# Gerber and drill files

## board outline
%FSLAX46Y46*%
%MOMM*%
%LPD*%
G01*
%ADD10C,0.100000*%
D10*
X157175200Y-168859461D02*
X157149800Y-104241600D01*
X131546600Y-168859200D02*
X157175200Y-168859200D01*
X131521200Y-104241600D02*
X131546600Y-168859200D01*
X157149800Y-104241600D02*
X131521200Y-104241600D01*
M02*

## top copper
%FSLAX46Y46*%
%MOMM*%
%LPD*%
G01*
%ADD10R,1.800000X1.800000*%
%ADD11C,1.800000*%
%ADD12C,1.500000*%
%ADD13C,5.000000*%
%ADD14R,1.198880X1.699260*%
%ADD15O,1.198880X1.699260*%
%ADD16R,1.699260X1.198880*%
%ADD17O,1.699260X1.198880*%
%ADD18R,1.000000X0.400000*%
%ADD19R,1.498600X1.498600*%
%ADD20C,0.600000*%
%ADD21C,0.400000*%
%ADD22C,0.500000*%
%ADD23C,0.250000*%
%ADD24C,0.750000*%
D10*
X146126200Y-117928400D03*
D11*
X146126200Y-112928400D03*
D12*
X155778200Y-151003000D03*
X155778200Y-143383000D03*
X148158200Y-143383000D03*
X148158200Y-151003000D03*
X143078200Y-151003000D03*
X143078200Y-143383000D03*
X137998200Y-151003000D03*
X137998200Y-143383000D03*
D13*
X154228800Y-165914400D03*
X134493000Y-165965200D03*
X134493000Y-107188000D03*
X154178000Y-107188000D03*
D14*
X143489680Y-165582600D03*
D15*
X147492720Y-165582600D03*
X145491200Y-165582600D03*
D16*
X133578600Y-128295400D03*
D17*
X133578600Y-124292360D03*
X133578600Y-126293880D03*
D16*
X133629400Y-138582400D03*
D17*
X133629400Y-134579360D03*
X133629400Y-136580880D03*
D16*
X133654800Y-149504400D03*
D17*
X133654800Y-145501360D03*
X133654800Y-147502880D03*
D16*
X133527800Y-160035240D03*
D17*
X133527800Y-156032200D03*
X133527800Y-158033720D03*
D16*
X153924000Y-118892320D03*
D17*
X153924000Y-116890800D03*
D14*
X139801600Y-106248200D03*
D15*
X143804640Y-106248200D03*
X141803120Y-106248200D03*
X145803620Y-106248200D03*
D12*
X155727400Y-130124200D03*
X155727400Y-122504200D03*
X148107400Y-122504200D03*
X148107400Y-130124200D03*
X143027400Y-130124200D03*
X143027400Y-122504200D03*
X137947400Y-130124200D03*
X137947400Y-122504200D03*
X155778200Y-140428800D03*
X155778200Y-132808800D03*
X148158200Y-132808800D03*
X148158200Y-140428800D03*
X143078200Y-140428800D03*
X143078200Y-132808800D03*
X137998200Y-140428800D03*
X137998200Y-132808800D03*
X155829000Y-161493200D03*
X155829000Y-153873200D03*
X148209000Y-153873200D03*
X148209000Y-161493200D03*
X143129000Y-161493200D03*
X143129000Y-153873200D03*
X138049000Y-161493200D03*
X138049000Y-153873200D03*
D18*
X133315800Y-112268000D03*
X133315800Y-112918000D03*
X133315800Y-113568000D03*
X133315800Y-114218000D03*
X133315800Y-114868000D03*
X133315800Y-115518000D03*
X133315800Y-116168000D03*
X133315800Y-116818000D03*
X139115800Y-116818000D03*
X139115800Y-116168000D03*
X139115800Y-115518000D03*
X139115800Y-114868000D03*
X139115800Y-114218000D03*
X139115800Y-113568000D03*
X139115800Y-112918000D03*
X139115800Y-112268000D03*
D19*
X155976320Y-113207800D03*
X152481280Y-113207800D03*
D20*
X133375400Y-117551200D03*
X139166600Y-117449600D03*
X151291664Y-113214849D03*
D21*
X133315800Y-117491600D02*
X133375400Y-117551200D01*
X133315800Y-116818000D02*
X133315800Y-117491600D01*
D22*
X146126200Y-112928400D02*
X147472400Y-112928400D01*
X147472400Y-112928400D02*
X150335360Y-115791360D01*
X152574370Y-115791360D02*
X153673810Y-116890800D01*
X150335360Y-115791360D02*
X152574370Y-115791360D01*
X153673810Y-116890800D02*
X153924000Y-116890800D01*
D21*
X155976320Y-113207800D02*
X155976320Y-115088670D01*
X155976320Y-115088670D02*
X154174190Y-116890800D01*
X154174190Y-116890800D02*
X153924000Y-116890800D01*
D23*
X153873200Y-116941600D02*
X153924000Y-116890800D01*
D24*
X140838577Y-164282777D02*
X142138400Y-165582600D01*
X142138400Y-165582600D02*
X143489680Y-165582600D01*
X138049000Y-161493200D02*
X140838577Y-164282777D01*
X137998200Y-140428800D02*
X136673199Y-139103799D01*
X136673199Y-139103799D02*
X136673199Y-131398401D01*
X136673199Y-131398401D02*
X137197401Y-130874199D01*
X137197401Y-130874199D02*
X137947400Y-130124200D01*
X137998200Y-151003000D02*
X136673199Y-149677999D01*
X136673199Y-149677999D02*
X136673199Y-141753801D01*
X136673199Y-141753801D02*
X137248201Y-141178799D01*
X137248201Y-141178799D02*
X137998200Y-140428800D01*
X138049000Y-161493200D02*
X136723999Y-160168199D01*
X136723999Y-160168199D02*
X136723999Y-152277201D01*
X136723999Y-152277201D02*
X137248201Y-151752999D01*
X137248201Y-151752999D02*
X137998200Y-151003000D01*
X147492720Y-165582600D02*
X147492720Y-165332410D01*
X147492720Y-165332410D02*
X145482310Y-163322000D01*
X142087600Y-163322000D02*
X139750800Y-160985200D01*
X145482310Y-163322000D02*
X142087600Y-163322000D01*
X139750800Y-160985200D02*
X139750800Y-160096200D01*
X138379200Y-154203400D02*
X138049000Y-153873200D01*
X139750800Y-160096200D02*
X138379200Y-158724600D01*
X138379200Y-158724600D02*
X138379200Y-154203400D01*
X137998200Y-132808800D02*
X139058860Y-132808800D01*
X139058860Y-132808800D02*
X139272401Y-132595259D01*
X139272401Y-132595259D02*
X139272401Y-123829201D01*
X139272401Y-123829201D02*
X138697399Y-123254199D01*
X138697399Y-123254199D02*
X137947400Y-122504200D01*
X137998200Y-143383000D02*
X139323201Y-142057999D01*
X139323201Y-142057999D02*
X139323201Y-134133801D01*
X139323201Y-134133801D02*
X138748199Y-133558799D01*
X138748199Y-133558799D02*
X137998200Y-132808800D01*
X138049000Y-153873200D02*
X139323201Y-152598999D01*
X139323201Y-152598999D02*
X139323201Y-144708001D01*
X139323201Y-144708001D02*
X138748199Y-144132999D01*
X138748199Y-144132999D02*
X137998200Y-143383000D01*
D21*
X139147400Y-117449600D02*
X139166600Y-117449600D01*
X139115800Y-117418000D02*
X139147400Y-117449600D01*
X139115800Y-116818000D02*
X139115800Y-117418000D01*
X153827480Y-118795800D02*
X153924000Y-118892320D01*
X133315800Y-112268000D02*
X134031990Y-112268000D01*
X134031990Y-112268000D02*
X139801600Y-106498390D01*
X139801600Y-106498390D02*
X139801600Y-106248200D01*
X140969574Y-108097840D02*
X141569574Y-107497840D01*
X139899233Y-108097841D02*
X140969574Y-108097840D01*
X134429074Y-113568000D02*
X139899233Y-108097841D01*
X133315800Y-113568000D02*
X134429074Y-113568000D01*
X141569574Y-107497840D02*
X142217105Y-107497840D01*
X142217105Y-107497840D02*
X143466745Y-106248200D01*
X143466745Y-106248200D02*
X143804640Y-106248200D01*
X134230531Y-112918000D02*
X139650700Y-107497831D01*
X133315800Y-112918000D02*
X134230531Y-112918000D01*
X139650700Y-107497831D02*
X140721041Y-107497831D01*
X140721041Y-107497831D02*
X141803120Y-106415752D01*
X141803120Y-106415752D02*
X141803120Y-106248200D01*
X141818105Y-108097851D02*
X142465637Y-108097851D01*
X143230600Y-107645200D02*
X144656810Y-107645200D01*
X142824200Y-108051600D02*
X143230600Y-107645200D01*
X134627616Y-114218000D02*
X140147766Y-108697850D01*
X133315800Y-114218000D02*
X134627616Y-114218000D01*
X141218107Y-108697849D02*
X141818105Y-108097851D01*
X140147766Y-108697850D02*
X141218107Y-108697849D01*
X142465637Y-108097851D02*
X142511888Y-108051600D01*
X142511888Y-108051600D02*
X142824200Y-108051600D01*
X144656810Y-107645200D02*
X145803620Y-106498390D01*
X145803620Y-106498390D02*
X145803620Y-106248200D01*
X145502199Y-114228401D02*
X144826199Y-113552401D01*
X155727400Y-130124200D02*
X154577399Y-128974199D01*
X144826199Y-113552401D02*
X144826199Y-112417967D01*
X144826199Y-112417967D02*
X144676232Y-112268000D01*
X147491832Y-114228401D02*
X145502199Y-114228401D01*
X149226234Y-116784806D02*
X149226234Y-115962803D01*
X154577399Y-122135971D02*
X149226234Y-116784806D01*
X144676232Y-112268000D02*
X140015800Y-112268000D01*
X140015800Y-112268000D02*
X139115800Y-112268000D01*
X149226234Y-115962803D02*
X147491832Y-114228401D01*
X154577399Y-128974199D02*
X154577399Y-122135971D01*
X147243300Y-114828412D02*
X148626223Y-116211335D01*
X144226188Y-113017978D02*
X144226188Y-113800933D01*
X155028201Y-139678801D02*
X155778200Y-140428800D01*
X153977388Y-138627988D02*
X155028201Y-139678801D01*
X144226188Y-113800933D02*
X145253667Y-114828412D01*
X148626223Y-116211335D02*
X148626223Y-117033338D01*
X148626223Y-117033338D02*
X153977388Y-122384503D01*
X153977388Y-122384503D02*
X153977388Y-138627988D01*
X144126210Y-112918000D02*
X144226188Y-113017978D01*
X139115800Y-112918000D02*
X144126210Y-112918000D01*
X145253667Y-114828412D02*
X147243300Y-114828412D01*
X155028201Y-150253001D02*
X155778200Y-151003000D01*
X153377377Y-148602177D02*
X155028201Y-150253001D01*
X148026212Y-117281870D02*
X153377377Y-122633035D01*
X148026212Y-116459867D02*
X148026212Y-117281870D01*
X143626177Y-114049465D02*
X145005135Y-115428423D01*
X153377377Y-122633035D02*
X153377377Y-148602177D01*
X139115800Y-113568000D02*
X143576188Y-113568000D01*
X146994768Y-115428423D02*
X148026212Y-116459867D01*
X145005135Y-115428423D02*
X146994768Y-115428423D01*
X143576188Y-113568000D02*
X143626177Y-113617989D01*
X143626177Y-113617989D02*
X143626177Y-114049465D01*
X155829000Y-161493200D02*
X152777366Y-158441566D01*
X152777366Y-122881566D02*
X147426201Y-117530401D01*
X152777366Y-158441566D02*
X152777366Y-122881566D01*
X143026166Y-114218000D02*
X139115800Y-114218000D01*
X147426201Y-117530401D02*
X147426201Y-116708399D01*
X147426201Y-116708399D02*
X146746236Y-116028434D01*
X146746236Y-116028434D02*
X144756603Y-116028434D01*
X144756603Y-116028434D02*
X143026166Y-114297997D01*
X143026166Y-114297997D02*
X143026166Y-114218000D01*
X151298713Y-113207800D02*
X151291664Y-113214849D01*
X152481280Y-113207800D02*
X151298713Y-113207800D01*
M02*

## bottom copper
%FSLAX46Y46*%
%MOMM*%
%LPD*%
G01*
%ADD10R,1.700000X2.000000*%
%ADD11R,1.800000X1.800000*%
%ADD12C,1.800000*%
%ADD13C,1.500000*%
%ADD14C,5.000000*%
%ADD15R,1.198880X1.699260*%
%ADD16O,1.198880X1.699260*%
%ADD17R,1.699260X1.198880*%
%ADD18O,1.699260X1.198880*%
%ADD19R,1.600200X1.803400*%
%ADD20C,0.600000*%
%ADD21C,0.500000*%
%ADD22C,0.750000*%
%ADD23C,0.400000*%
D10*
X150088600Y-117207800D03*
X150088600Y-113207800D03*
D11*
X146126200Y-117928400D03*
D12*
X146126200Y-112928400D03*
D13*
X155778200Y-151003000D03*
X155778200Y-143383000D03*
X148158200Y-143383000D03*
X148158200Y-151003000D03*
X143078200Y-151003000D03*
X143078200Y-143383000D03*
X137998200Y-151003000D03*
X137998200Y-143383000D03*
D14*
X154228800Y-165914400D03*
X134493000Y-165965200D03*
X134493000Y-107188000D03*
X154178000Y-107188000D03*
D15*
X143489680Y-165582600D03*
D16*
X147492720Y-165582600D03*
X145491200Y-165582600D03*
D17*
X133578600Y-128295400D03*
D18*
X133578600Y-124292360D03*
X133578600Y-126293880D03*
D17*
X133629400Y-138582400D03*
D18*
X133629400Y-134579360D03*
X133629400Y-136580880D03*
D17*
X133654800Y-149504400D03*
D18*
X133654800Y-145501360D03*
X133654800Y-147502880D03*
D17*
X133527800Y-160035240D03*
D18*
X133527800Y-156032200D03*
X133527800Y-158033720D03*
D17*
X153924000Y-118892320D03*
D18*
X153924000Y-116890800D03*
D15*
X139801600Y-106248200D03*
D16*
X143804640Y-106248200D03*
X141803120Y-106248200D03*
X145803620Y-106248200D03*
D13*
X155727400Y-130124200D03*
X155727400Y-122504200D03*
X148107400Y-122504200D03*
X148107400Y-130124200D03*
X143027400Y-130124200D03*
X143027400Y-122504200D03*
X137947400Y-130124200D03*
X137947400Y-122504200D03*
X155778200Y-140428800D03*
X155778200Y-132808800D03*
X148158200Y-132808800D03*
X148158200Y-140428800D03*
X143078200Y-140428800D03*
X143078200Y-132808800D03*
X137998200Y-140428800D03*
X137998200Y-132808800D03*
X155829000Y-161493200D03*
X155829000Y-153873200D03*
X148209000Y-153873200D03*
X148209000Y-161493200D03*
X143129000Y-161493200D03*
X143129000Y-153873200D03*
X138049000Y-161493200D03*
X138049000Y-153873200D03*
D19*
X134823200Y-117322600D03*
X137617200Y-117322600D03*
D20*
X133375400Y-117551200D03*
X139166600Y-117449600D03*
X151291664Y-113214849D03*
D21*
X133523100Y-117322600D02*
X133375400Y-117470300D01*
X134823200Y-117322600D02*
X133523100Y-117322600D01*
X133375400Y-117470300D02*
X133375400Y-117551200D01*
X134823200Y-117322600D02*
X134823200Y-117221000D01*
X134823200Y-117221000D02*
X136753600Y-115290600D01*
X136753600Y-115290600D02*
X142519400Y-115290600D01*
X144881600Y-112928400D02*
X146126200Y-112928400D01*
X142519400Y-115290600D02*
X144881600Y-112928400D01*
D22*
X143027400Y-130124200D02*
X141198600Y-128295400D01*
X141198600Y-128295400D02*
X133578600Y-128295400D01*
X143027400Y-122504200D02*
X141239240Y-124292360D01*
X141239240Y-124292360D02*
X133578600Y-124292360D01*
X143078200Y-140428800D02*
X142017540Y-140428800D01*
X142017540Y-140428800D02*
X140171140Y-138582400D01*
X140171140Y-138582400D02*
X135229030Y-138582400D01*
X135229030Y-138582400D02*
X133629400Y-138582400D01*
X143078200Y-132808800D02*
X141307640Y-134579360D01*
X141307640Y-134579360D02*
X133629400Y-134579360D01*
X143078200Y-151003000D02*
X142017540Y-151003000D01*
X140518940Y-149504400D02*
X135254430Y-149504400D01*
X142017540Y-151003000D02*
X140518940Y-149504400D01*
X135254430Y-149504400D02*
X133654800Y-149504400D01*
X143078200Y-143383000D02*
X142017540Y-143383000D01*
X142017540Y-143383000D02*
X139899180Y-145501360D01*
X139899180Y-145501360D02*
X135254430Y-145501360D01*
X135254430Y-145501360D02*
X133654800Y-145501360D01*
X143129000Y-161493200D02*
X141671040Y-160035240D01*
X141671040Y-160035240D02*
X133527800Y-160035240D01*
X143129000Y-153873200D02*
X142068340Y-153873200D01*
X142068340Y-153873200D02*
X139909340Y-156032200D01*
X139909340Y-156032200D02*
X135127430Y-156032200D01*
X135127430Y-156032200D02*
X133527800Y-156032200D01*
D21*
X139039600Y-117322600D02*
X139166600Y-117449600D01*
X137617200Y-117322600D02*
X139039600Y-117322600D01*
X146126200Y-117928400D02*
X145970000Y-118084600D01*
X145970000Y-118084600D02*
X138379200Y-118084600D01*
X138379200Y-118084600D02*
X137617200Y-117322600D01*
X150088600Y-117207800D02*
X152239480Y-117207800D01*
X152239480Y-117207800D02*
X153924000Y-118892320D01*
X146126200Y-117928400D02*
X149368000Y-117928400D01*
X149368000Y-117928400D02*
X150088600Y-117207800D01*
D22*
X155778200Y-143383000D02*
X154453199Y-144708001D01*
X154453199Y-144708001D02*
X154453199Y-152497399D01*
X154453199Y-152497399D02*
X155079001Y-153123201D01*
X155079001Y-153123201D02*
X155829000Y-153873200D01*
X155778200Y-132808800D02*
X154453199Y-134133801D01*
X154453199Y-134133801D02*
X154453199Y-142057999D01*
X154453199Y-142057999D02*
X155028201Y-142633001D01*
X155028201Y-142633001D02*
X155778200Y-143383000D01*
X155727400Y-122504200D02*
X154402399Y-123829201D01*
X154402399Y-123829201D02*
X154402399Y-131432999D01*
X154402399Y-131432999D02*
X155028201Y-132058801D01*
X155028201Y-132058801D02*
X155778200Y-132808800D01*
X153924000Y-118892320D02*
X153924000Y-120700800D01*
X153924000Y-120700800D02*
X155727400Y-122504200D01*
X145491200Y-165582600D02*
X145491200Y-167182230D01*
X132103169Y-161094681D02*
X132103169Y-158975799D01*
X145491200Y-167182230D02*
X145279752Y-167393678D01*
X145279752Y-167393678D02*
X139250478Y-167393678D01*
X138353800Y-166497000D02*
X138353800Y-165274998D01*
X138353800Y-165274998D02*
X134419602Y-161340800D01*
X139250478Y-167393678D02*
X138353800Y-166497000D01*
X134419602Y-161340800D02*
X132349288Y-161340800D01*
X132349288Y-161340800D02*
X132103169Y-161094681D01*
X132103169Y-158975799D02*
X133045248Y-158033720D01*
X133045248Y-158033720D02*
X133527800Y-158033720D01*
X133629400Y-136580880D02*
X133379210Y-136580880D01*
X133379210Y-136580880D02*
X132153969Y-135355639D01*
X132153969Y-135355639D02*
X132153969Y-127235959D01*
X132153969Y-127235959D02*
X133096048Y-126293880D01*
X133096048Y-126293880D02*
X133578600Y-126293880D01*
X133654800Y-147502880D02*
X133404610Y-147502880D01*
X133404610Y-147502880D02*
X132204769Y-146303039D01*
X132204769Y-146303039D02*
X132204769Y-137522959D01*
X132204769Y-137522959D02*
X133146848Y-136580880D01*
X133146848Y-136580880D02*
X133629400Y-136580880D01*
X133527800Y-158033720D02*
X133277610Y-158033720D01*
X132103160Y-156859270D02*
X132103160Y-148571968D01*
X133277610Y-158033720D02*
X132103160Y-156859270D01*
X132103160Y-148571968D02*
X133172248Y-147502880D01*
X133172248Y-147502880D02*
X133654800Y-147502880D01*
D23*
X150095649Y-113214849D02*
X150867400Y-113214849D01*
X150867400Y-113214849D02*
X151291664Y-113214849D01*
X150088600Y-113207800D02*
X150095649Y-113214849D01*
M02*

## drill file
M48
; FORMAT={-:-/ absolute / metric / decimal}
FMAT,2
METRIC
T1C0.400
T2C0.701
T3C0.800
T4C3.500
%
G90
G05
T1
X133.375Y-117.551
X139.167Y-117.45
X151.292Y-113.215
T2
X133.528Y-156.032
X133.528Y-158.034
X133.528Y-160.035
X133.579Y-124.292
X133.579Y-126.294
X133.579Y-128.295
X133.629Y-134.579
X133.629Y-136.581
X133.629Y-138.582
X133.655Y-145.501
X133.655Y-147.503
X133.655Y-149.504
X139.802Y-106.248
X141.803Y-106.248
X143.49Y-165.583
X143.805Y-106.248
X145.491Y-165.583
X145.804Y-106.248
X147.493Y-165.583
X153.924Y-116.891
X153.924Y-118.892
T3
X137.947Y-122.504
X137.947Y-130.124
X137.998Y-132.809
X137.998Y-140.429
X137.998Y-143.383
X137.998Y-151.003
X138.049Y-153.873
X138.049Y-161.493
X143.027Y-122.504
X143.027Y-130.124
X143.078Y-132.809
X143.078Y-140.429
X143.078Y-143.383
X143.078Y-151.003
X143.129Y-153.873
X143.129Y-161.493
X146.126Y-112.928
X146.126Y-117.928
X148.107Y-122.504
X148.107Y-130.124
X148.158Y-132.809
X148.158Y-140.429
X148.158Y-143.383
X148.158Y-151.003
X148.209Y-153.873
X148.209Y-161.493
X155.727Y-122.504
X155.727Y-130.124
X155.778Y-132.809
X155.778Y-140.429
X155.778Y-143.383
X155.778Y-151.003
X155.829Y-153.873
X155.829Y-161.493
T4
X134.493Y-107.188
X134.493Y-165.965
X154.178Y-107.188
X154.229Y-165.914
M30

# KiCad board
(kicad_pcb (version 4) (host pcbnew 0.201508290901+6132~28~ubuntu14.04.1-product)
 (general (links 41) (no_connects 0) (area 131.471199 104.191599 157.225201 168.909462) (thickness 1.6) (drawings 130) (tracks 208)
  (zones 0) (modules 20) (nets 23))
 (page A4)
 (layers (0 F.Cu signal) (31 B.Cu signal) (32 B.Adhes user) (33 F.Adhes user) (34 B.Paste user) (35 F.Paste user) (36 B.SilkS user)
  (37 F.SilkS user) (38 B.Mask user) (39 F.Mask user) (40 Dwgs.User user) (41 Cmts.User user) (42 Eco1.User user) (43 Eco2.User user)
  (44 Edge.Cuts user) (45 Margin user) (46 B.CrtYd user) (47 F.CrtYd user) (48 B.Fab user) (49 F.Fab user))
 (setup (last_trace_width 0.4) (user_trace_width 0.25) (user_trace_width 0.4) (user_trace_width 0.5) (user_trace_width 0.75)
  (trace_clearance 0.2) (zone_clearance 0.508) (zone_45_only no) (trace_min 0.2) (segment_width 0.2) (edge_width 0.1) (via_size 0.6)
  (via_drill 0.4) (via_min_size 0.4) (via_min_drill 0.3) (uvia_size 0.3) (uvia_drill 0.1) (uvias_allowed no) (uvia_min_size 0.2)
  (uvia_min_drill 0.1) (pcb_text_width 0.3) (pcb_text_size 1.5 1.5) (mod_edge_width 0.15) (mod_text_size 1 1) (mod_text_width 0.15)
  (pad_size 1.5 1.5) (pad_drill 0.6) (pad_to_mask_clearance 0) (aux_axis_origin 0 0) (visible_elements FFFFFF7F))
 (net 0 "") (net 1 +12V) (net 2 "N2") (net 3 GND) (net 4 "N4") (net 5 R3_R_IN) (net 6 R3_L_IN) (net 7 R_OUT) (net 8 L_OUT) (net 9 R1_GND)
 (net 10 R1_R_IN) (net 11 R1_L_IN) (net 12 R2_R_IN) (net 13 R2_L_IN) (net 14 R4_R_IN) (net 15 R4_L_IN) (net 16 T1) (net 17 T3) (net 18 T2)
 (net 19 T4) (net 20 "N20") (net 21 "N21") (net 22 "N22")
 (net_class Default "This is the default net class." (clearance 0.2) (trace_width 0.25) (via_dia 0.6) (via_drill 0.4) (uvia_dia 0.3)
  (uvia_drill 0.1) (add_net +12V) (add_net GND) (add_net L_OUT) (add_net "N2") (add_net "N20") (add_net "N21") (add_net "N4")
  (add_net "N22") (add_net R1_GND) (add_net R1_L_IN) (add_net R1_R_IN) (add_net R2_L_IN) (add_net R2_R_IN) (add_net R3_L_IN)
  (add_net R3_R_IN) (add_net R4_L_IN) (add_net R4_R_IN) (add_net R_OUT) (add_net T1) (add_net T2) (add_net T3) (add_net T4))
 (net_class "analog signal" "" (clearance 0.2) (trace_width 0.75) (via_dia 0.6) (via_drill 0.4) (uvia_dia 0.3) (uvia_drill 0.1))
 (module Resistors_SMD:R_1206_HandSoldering (layer B.Cu) (at 150.0886 115.2078 90)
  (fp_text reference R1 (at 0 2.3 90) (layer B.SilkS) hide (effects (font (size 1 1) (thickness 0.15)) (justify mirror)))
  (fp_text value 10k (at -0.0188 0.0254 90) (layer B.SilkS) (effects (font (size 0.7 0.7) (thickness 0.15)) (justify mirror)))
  (pad 1 smd rect (at -2 0 90) (size 2 1.7) (layers B.Cu B.Paste B.Mask) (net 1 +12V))
  (pad 2 smd rect (at 2 0 90) (size 2 1.7) (layers B.Cu B.Paste B.Mask) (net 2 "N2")))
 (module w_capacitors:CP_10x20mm (layer F.Cu) (at 146.1262 115.4284)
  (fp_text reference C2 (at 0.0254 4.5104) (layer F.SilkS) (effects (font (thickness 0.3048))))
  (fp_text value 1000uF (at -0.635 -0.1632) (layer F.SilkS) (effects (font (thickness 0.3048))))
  (pad 1 thru_hole rect (at 0 2.5) (size 1.8 1.8) (drill 0.8) (layers *.Cu *.Mask F.SilkS) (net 1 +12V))
  (pad 2 thru_hole circle (at 0 -2.5) (size 1.8 1.8) (drill 0.8) (layers *.Cu *.Mask F.SilkS) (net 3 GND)))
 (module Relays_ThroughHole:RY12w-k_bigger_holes (layer F.Cu) (at 156.9782 152.103 180)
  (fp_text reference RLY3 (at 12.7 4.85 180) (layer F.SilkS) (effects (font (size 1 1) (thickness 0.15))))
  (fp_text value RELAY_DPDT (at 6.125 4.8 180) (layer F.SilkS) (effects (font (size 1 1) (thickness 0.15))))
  (pad 1 thru_hole circle (at 1.2 1.1 180) (size 1.5 1.5) (drill 0.8) (layers *.Cu *.Mask F.SilkS) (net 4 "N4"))
  (pad 8 thru_hole circle (at 1.2 8.72 180) (size 1.5 1.5) (drill 0.8) (layers *.Cu *.Mask F.SilkS) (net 1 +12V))
  (pad 7 thru_hole circle (at 8.82 8.72 180) (size 1.5 1.5) (drill 0.8) (layers *.Cu *.Mask F.SilkS))
  (pad 2 thru_hole circle (at 8.82 1.1 180) (size 1.5 1.5) (drill 0.8) (layers *.Cu *.Mask F.SilkS))
  (pad 3 thru_hole circle (at 13.9 1.1 180) (size 1.5 1.5) (drill 0.8) (layers *.Cu *.Mask F.SilkS) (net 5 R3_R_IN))
  (pad 6 thru_hole circle (at 13.9 8.72 180) (size 1.5 1.5) (drill 0.8) (layers *.Cu *.Mask F.SilkS) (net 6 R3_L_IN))
  (pad 4 thru_hole circle (at 18.98 1.1 180) (size 1.5 1.5) (drill 0.8) (layers *.Cu *.Mask F.SilkS) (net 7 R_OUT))
  (pad 5 thru_hole circle (at 18.98 8.72 180) (size 1.5 1.5) (drill 0.8) (layers *.Cu *.Mask F.SilkS) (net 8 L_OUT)))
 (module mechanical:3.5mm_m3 (layer F.Cu) (at 154.2288 166.0144)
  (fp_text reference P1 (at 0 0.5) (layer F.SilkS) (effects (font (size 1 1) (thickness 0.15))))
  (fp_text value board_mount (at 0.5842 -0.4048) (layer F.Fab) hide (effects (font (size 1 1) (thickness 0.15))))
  (pad 1 thru_hole circle (at 0 -0.1) (size 5 5) (drill 3.5) (layers *.Cu *.Mask F.SilkS)))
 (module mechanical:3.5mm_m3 (layer F.Cu) (at 134.493 166.0652)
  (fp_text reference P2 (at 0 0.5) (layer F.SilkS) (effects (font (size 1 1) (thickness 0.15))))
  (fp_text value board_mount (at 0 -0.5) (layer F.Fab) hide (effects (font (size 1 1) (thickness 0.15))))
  (pad 1 thru_hole circle (at 0 -0.1) (size 5 5) (drill 3.5) (layers *.Cu *.Mask F.SilkS)))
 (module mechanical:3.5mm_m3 (layer F.Cu) (at 134.493 107.288)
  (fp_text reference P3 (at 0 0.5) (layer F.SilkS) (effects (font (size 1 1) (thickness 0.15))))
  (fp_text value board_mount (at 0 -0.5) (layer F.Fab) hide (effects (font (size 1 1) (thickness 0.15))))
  (pad 1 thru_hole circle (at 0 -0.1) (size 5 5) (drill 3.5) (layers *.Cu *.Mask F.SilkS)))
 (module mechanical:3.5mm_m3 (layer F.Cu) (at 154.178 107.288)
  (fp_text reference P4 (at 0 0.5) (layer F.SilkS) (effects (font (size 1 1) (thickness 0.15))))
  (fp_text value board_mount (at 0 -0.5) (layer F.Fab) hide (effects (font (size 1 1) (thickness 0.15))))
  (pad 1 thru_hole circle (at 0 -0.1) (size 5 5) (drill 3.5) (layers *.Cu *.Mask F.SilkS)))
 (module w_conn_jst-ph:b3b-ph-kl (layer F.Cu) (at 145.4912 165.5826)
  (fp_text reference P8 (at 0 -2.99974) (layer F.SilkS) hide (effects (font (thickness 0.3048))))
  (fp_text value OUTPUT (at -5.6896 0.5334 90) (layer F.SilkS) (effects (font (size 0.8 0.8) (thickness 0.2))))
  (pad 1 thru_hole rect (at -2.00152 0) (size 1.19888 1.69926) (drill 0.70104) (layers *.Cu *.Mask F.SilkS) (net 7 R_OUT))
  (pad 3 thru_hole oval (at 2.00152 0) (size 1.19888 1.69926) (drill 0.70104) (layers *.Cu *.Mask F.SilkS) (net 8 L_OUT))
  (pad 2 thru_hole oval (at 0 0) (size 1.19888 1.69926) (drill 0.70104) (layers *.Cu *.Mask F.SilkS) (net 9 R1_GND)))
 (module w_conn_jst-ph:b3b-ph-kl (layer F.Cu) (at 133.5786 126.29388 90)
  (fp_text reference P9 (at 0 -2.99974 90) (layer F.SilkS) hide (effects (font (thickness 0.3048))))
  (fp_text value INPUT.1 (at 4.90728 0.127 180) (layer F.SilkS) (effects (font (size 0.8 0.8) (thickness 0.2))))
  (pad 1 thru_hole rect (at -2.00152 0 90) (size 1.19888 1.69926) (drill 0.70104) (layers *.Cu *.Mask F.SilkS) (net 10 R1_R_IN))
  (pad 3 thru_hole oval (at 2.00152 0 90) (size 1.19888 1.69926) (drill 0.70104) (layers *.Cu *.Mask F.SilkS) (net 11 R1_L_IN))
  (pad 2 thru_hole oval (at 0 0 90) (size 1.19888 1.69926) (drill 0.70104) (layers *.Cu *.Mask F.SilkS) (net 9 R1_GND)))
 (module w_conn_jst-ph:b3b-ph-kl (layer F.Cu) (at 133.6294 136.58088 90)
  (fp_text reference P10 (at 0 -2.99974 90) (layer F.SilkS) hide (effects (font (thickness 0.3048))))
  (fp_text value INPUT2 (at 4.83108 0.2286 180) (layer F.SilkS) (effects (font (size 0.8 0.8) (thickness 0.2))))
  (pad 1 thru_hole rect (at -2.00152 0 90) (size 1.19888 1.69926) (drill 0.70104) (layers *.Cu *.Mask F.SilkS) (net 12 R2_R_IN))
  (pad 3 thru_hole oval (at 2.00152 0 90) (size 1.19888 1.69926) (drill 0.70104) (layers *.Cu *.Mask F.SilkS) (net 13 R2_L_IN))
  (pad 2 thru_hole oval (at 0 0 90) (size 1.19888 1.69926) (drill 0.70104) (layers *.Cu *.Mask F.SilkS) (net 9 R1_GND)))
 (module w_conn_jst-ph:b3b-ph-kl (layer F.Cu) (at 133.6548 147.50288 90)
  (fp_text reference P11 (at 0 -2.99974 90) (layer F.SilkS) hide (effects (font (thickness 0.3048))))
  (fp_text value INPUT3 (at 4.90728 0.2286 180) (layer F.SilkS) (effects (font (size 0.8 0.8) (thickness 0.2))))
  (pad 1 thru_hole rect (at -2.00152 0 90) (size 1.19888 1.69926) (drill 0.70104) (layers *.Cu *.Mask F.SilkS) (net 5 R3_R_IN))
  (pad 3 thru_hole oval (at 2.00152 0 90) (size 1.19888 1.69926) (drill 0.70104) (layers *.Cu *.Mask F.SilkS) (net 6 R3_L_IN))
  (pad 2 thru_hole oval (at 0 0 90) (size 1.19888 1.69926) (drill 0.70104) (layers *.Cu *.Mask F.SilkS) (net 9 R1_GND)))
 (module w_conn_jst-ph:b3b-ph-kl (layer F.Cu) (at 133.5278 158.03372 90)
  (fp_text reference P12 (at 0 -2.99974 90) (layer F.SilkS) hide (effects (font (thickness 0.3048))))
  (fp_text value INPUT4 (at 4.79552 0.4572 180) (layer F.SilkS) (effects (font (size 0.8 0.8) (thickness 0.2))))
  (pad 1 thru_hole rect (at -2.00152 0 90) (size 1.19888 1.69926) (drill 0.70104) (layers *.Cu *.Mask F.SilkS) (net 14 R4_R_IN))
  (pad 3 thru_hole oval (at 2.00152 0 90) (size 1.19888 1.69926) (drill 0.70104) (layers *.Cu *.Mask F.SilkS) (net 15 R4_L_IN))
  (pad 2 thru_hole oval (at 0 0 90) (size 1.19888 1.69926) (drill 0.70104) (layers *.Cu *.Mask F.SilkS) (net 9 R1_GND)))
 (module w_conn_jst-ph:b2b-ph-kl (layer F.Cu) (at 153.924 117.89156 90)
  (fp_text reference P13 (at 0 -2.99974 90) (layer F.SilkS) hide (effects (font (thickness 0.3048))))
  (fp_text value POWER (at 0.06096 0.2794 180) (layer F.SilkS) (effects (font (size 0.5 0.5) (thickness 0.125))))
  (pad 1 thru_hole rect (at -1.00076 0 90) (size 1.19888 1.69926) (drill 0.70104) (layers *.Cu *.Mask F.SilkS) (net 1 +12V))
  (pad 2 thru_hole oval (at 1.00076 0 90) (size 1.19888 1.69926) (drill 0.70104) (layers *.Cu *.Mask F.SilkS) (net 3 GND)))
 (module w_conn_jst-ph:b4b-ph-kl (layer F.Cu) (at 142.80388 106.2482)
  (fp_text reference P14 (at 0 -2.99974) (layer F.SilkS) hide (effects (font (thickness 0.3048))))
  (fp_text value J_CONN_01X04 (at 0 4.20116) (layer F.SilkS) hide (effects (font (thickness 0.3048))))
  (pad 1 thru_hole rect (at -3.00228 0) (size 1.19888 1.69926) (drill 0.70104) (layers *.Cu *.Mask F.SilkS) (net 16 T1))
  (pad 3 thru_hole oval (at 1.00076 0) (size 1.19888 1.69926) (drill 0.70104) (layers *.Cu *.Mask F.SilkS) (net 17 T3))
  (pad 2 thru_hole oval (at -1.00076 0) (size 1.19888 1.69926) (drill 0.70104) (layers *.Cu *.Mask F.SilkS) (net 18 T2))
  (pad 4 thru_hole oval (at 2.99974 0) (size 1.19888 1.69926) (drill 0.70104) (layers *.Cu *.Mask F.SilkS) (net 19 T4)))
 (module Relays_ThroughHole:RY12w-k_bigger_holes (layer F.Cu) (at 156.9274 131.2242 180)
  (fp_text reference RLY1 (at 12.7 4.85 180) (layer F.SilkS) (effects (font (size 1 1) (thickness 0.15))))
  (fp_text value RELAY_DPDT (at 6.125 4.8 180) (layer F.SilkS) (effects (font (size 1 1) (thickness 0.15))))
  (pad 1 thru_hole circle (at 1.2 1.1 180) (size 1.5 1.5) (drill 0.8) (layers *.Cu *.Mask F.SilkS) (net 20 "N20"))
  (pad 8 thru_hole circle (at 1.2 8.72 180) (size 1.5 1.5) (drill 0.8) (layers *.Cu *.Mask F.SilkS) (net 1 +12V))
  (pad 7 thru_hole circle (at 8.82 8.72 180) (size 1.5 1.5) (drill 0.8) (layers *.Cu *.Mask F.SilkS))
  (pad 2 thru_hole circle (at 8.82 1.1 180) (size 1.5 1.5) (drill 0.8) (layers *.Cu *.Mask F.SilkS))
  (pad 3 thru_hole circle (at 13.9 1.1 180) (size 1.5 1.5) (drill 0.8) (layers *.Cu *.Mask F.SilkS) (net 10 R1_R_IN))
  (pad 6 thru_hole circle (at 13.9 8.72 180) (size 1.5 1.5) (drill 0.8) (layers *.Cu *.Mask F.SilkS) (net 11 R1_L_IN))
  (pad 4 thru_hole circle (at 18.98 1.1 180) (size 1.5 1.5) (drill 0.8) (layers *.Cu *.Mask F.SilkS) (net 7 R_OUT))
  (pad 5 thru_hole circle (at 18.98 8.72 180) (size 1.5 1.5) (drill 0.8) (layers *.Cu *.Mask F.SilkS) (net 8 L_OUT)))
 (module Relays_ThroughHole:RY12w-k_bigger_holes (layer F.Cu) (at 156.9782 141.5288 180)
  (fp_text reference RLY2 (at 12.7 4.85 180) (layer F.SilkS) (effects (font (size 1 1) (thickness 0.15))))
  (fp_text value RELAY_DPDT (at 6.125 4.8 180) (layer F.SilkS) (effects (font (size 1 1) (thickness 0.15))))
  (pad 1 thru_hole circle (at 1.2 1.1 180) (size 1.5 1.5) (drill 0.8) (layers *.Cu *.Mask F.SilkS) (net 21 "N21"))
  (pad 8 thru_hole circle (at 1.2 8.72 180) (size 1.5 1.5) (drill 0.8) (layers *.Cu *.Mask F.SilkS) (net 1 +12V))
  (pad 7 thru_hole circle (at 8.82 8.72 180) (size 1.5 1.5) (drill 0.8) (layers *.Cu *.Mask F.SilkS))
  (pad 2 thru_hole circle (at 8.82 1.1 180) (size 1.5 1.5) (drill 0.8) (layers *.Cu *.Mask F.SilkS))
  (pad 3 thru_hole circle (at 13.9 1.1 180) (size 1.5 1.5) (drill 0.8) (layers *.Cu *.Mask F.SilkS) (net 12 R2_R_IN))
  (pad 6 thru_hole circle (at 13.9 8.72 180) (size 1.5 1.5) (drill 0.8) (layers *.Cu *.Mask F.SilkS) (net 13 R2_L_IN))
  (pad 4 thru_hole circle (at 18.98 1.1 180) (size 1.5 1.5) (drill 0.8) (layers *.Cu *.Mask F.SilkS) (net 7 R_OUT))
  (pad 5 thru_hole circle (at 18.98 8.72 180) (size 1.5 1.5) (drill 0.8) (layers *.Cu *.Mask F.SilkS) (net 8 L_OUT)))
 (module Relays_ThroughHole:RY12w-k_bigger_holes (layer F.Cu) (at 157.029 162.5932 180)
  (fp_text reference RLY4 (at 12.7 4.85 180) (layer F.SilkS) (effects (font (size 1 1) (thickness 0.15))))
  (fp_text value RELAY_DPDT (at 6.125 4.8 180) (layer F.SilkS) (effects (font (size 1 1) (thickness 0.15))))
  (pad 1 thru_hole circle (at 1.2 1.1 180) (size 1.5 1.5) (drill 0.8) (layers *.Cu *.Mask F.SilkS) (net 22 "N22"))
  (pad 8 thru_hole circle (at 1.2 8.72 180) (size 1.5 1.5) (drill 0.8) (layers *.Cu *.Mask F.SilkS) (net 1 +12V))
  (pad 7 thru_hole circle (at 8.82 8.72 180) (size 1.5 1.5) (drill 0.8) (layers *.Cu *.Mask F.SilkS))
  (pad 2 thru_hole circle (at 8.82 1.1 180) (size 1.5 1.5) (drill 0.8) (layers *.Cu *.Mask F.SilkS))
  (pad 3 thru_hole circle (at 13.9 1.1 180) (size 1.5 1.5) (drill 0.8) (layers *.Cu *.Mask F.SilkS) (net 14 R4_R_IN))
  (pad 6 thru_hole circle (at 13.9 8.72 180) (size 1.5 1.5) (drill 0.8) (layers *.Cu *.Mask F.SilkS) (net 15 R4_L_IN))
  (pad 4 thru_hole circle (at 18.98 1.1 180) (size 1.5 1.5) (drill 0.8) (layers *.Cu *.Mask F.SilkS) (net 7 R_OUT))
  (pad 5 thru_hole circle (at 18.98 8.72 180) (size 1.5 1.5) (drill 0.8) (layers *.Cu *.Mask F.SilkS) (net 8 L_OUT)))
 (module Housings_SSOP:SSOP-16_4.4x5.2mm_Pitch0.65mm (layer F.Cu) (at 136.2158 114.543)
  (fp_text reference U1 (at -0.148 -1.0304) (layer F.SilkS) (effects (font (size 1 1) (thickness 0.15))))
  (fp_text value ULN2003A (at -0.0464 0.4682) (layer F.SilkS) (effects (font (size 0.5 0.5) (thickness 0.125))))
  (pad 1 smd rect (at -2.9 -2.275) (size 1 0.4) (layers F.Cu F.Paste F.Mask) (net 16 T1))
  (pad 2 smd rect (at -2.9 -1.625) (size 1 0.4) (layers F.Cu F.Paste F.Mask) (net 18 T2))
  (pad 3 smd rect (at -2.9 -0.975) (size 1 0.4) (layers F.Cu F.Paste F.Mask) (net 17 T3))
  (pad 4 smd rect (at -2.9 -0.325) (size 1 0.4) (layers F.Cu F.Paste F.Mask) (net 19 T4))
  (pad 5 smd rect (at -2.9 0.325) (size 1 0.4) (layers F.Cu F.Paste F.Mask))
  (pad 6 smd rect (at -2.9 0.975) (size 1 0.4) (layers F.Cu F.Paste F.Mask))
  (pad 7 smd rect (at -2.9 1.625) (size 1 0.4) (layers F.Cu F.Paste F.Mask))
  (pad 8 smd rect (at -2.9 2.275) (size 1 0.4) (layers F.Cu F.Paste F.Mask) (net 3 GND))
  (pad 9 smd rect (at 2.9 2.275) (size 1 0.4) (layers F.Cu F.Paste F.Mask) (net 1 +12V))
  (pad 10 smd rect (at 2.9 1.625) (size 1 0.4) (layers F.Cu F.Paste F.Mask))
  (pad 11 smd rect (at 2.9 0.975) (size 1 0.4) (layers F.Cu F.Paste F.Mask))
  (pad 12 smd rect (at 2.9 0.325) (size 1 0.4) (layers F.Cu F.Paste F.Mask))
  (pad 13 smd rect (at 2.9 -0.325) (size 1 0.4) (layers F.Cu F.Paste F.Mask) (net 22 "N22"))
  (pad 14 smd rect (at 2.9 -0.975) (size 1 0.4) (layers F.Cu F.Paste F.Mask) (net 4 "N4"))
  (pad 15 smd rect (at 2.9 -1.625) (size 1 0.4) (layers F.Cu F.Paste F.Mask) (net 21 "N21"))
  (pad 16 smd rect (at 2.9 -2.275) (size 1 0.4) (layers F.Cu F.Paste F.Mask) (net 20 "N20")))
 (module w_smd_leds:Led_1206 (layer F.Cu) (at 154.2288 113.2078 180)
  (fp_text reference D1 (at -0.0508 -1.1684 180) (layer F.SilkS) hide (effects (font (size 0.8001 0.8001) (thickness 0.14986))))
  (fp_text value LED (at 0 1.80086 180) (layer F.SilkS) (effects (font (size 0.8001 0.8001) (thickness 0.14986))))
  (pad 1 smd rect (at -1.74752 0 180) (size 1.4986 1.4986) (layers F.Cu F.Paste F.Mask) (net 3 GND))
  (pad 2 smd rect (at 1.74752 0 180) (size 1.4986 1.4986) (layers F.Cu F.Paste F.Mask) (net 2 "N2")))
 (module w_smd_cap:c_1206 (layer B.Cu) (at 136.2202 117.3226 180)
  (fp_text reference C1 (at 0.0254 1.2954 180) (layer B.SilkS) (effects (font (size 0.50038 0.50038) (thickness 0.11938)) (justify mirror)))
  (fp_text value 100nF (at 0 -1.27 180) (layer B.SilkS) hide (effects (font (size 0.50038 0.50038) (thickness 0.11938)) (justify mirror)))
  (pad 1 smd rect (at 1.397 0 180) (size 1.6002 1.8034) (layers B.Cu B.Paste B.Mask) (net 3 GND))
  (pad 2 smd rect (at -1.397 0 180) (size 1.6002 1.8034) (layers B.Cu B.Paste B.Mask) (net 1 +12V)))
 (gr_line (start 157.1752 168.859461) (end 157.1498 104.2416) (layer Edge.Cuts) (width 0.1))
 (gr_line (start 131.5466 168.8592) (end 157.1752 168.8592) (layer Edge.Cuts) (width 0.1))
 (gr_line (start 131.5212 104.2416) (end 131.5466 168.8592) (layer Edge.Cuts) (width 0.1))
 (gr_line (start 157.1498 104.2416) (end 131.5212 104.2416) (layer Edge.Cuts) (width 0.1))
 (segment (start 133.3158 117.4916) (end 133.3754 117.5512) (width 0.4) (layer F.Cu) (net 3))
 (segment (start 133.3158 116.818) (end 133.3158 117.4916) (width 0.4) (layer F.Cu) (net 3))
 (segment (start 133.5231 117.3226) (end 133.3754 117.4703) (width 0.5) (layer B.Cu) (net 3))
 (segment (start 134.8232 117.3226) (end 133.5231 117.3226) (width 0.5) (layer B.Cu) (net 3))
 (segment (start 133.3754 117.4703) (end 133.3754 117.5512) (width 0.5) (layer B.Cu) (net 3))
 (segment (start 134.8232 117.3226) (end 134.8232 117.221) (width 0.5) (layer B.Cu) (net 3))
 (segment (start 134.8232 117.221) (end 136.7536 115.2906) (width 0.5) (layer B.Cu) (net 3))
 (segment (start 136.7536 115.2906) (end 142.5194 115.2906) (width 0.5) (layer B.Cu) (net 3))
 (segment (start 144.8816 112.9284) (end 146.1262 112.9284) (width 0.5) (layer B.Cu) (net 3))
 (segment (start 142.5194 115.2906) (end 144.8816 112.9284) (width 0.5) (layer B.Cu) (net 3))
 (segment (start 146.1262 112.9284) (end 147.4724 112.9284) (width 0.5) (layer F.Cu) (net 3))
 (segment (start 147.4724 112.9284) (end 150.33536 115.79136) (width 0.5) (layer F.Cu) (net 3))
 (segment (start 152.57437 115.79136) (end 153.67381 116.8908) (width 0.5) (layer F.Cu) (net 3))
 (segment (start 150.33536 115.79136) (end 152.57437 115.79136) (width 0.5) (layer F.Cu) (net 3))
 (segment (start 153.67381 116.8908) (end 153.924 116.8908) (width 0.5) (layer F.Cu) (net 3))
 (segment (start 155.97632 113.2078) (end 155.97632 115.08867) (width 0.4) (layer F.Cu) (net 3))
 (segment (start 155.97632 115.08867) (end 154.17419 116.8908) (width 0.4) (layer F.Cu) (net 3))
 (segment (start 154.17419 116.8908) (end 153.924 116.8908) (width 0.4) (layer F.Cu) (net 3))
 (segment (start 153.8732 116.9416) (end 153.924 116.8908) (width 0.25) (layer F.Cu) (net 3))
 (segment (start 140.838577 164.282777) (end 142.1384 165.5826) (width 0.75) (layer F.Cu) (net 7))
 (segment (start 142.1384 165.5826) (end 143.48968 165.5826) (width 0.75) (layer F.Cu) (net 7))
 (segment (start 138.049 161.4932) (end 140.838577 164.282777) (width 0.75) (layer F.Cu) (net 7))
 (segment (start 137.9982 140.4288) (end 136.673199 139.103799) (width 0.75) (layer F.Cu) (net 7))
 (segment (start 136.673199 139.103799) (end 136.673199 131.398401) (width 0.75) (layer F.Cu) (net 7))
 (segment (start 136.673199 131.398401) (end 137.197401 130.874199) (width 0.75) (layer F.Cu) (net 7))
 (segment (start 137.197401 130.874199) (end 137.9474 130.1242) (width 0.75) (layer F.Cu) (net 7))
 (segment (start 137.9982 151.003) (end 136.673199 149.677999) (width 0.75) (layer F.Cu) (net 7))
 (segment (start 136.673199 149.677999) (end 136.673199 141.753801) (width 0.75) (layer F.Cu) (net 7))
 (segment (start 136.673199 141.753801) (end 137.248201 141.178799) (width 0.75) (layer F.Cu) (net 7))
 (segment (start 137.248201 141.178799) (end 137.9982 140.4288) (width 0.75) (layer F.Cu) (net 7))
 (segment (start 138.049 161.4932) (end 136.723999 160.168199) (width 0.75) (layer F.Cu) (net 7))
 (segment (start 136.723999 160.168199) (end 136.723999 152.277201) (width 0.75) (layer F.Cu) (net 7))
 (segment (start 136.723999 152.277201) (end 137.248201 151.752999) (width 0.75) (layer F.Cu) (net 7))
 (segment (start 137.248201 151.752999) (end 137.9982 151.003) (width 0.75) (layer F.Cu) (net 7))
 (segment (start 147.49272 165.5826) (end 147.49272 165.33241) (width 0.75) (layer F.Cu) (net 8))
 (segment (start 147.49272 165.33241) (end 145.48231 163.322) (width 0.75) (layer F.Cu) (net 8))
 (segment (start 142.0876 163.322) (end 139.7508 160.9852) (width 0.75) (layer F.Cu) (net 8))
 (segment (start 145.48231 163.322) (end 142.0876 163.322) (width 0.75) (layer F.Cu) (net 8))
 (segment (start 139.7508 160.9852) (end 139.7508 160.0962) (width 0.75) (layer F.Cu) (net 8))
 (segment (start 138.3792 154.2034) (end 138.049 153.8732) (width 0.75) (layer F.Cu) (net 8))
 (segment (start 139.7508 160.0962) (end 138.3792 158.7246) (width 0.75) (layer F.Cu) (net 8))
 (segment (start 138.3792 158.7246) (end 138.3792 154.2034) (width 0.75) (layer F.Cu) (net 8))
 (segment (start 137.9982 132.8088) (end 139.05886 132.8088) (width 0.75) (layer F.Cu) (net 8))
 (segment (start 139.05886 132.8088) (end 139.272401 132.595259) (width 0.75) (layer F.Cu) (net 8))
 (segment (start 139.272401 132.595259) (end 139.272401 123.829201) (width 0.75) (layer F.Cu) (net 8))
 (segment (start 139.272401 123.829201) (end 138.697399 123.254199) (width 0.75) (layer F.Cu) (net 8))
 (segment (start 138.697399 123.254199) (end 137.9474 122.5042) (width 0.75) (layer F.Cu) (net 8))
 (segment (start 137.9982 143.383) (end 139.323201 142.057999) (width 0.75) (layer F.Cu) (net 8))
 (segment (start 139.323201 142.057999) (end 139.323201 134.133801) (width 0.75) (layer F.Cu) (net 8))
 (segment (start 139.323201 134.133801) (end 138.748199 133.558799) (width 0.75) (layer F.Cu) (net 8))
 (segment (start 138.748199 133.558799) (end 137.9982 132.8088) (width 0.75) (layer F.Cu) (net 8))
 (segment (start 138.049 153.8732) (end 139.323201 152.598999) (width 0.75) (layer F.Cu) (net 8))
 (segment (start 139.323201 152.598999) (end 139.323201 144.708001) (width 0.75) (layer F.Cu) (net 8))
 (segment (start 139.323201 144.708001) (end 138.748199 144.132999) (width 0.75) (layer F.Cu) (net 8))
 (segment (start 138.748199 144.132999) (end 137.9982 143.383) (width 0.75) (layer F.Cu) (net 8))
 (segment (start 143.0274 130.1242) (end 141.1986 128.2954) (width 0.75) (layer B.Cu) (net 10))
 (segment (start 141.1986 128.2954) (end 133.5786 128.2954) (width 0.75) (layer B.Cu) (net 10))
 (segment (start 143.0274 122.5042) (end 141.23924 124.29236) (width 0.75) (layer B.Cu) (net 11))
 (segment (start 141.23924 124.29236) (end 133.5786 124.29236) (width 0.75) (layer B.Cu) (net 11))
 (segment (start 143.0782 140.4288) (end 142.01754 140.4288) (width 0.75) (layer B.Cu) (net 12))
 (segment (start 142.01754 140.4288) (end 140.17114 138.5824) (width 0.75) (layer B.Cu) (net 12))
 (segment (start 140.17114 138.5824) (end 135.22903 138.5824) (width 0.75) (layer B.Cu) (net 12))
 (segment (start 135.22903 138.5824) (end 133.6294 138.5824) (width 0.75) (layer B.Cu) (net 12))
 (segment (start 143.0782 132.8088) (end 141.30764 134.57936) (width 0.75) (layer B.Cu) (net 13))
 (segment (start 141.30764 134.57936) (end 133.6294 134.57936) (width 0.75) (layer B.Cu) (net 13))
 (segment (start 143.0782 151.003) (end 142.01754 151.003) (width 0.75) (layer B.Cu) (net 5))
 (segment (start 140.51894 149.5044) (end 135.25443 149.5044) (width 0.75) (layer B.Cu) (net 5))
 (segment (start 142.01754 151.003) (end 140.51894 149.5044) (width 0.75) (layer B.Cu) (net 5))
 (segment (start 135.25443 149.5044) (end 133.6548 149.5044) (width 0.75) (layer B.Cu) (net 5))
 (segment (start 143.0782 143.383) (end 142.01754 143.383) (width 0.75) (layer B.Cu) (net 6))
 (segment (start 142.01754 143.383) (end 139.89918 145.50136) (width 0.75) (layer B.Cu) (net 6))
 (segment (start 139.89918 145.50136) (end 135.25443 145.50136) (width 0.75) (layer B.Cu) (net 6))
 (segment (start 135.25443 145.50136) (end 133.6548 145.50136) (width 0.75) (layer B.Cu) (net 6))
 (segment (start 143.129 161.4932) (end 141.67104 160.03524) (width 0.75) (layer B.Cu) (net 14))
 (segment (start 141.67104 160.03524) (end 133.5278 160.03524) (width 0.75) (layer B.Cu) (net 14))
 (segment (start 143.129 153.8732) (end 142.06834 153.8732) (width 0.75) (layer B.Cu) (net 15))
 (segment (start 142.06834 153.8732) (end 139.90934 156.0322) (width 0.75) (layer B.Cu) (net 15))
 (segment (start 139.90934 156.0322) (end 135.12743 156.0322) (width 0.75) (layer B.Cu) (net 15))
 (segment (start 135.12743 156.0322) (end 133.5278 156.0322) (width 0.75) (layer B.Cu) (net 15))
 (segment (start 139.0396 117.3226) (end 139.1666 117.4496) (width 0.5) (layer B.Cu) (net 1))
 (segment (start 137.6172 117.3226) (end 139.0396 117.3226) (width 0.5) (layer B.Cu) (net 1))
 (segment (start 139.1474 117.4496) (end 139.1666 117.4496) (width 0.4) (layer F.Cu) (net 1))
 (segment (start 139.1158 117.418) (end 139.1474 117.4496) (width 0.4) (layer F.Cu) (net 1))
 (segment (start 139.1158 116.818) (end 139.1158 117.418) (width 0.4) (layer F.Cu) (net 1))
 (segment (start 146.1262 117.9284) (end 145.97 118.0846) (width 0.5) (layer B.Cu) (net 1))
 (segment (start 145.97 118.0846) (end 138.3792 118.0846) (width 0.5) (layer B.Cu) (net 1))
 (segment (start 138.3792 118.0846) (end 137.6172 117.3226) (width 0.5) (layer B.Cu) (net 1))
 (segment (start 150.0886 117.2078) (end 152.23948 117.2078) (width 0.5) (layer B.Cu) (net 1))
 (segment (start 152.23948 117.2078) (end 153.924 118.89232) (width 0.5) (layer B.Cu) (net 1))
 (segment (start 146.1262 117.9284) (end 149.368 117.9284) (width 0.5) (layer B.Cu) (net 1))
 (segment (start 149.368 117.9284) (end 150.0886 117.2078) (width 0.5) (layer B.Cu) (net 1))
 (segment (start 155.7782 143.383) (end 154.453199 144.708001) (width 0.75) (layer B.Cu) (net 1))
 (segment (start 154.453199 144.708001) (end 154.453199 152.497399) (width 0.75) (layer B.Cu) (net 1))
 (segment (start 154.453199 152.497399) (end 155.079001 153.123201) (width 0.75) (layer B.Cu) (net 1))
 (segment (start 155.079001 153.123201) (end 155.829 153.8732) (width 0.75) (layer B.Cu) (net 1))
 (segment (start 155.7782 132.8088) (end 154.453199 134.133801) (width 0.75) (layer B.Cu) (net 1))
 (segment (start 154.453199 134.133801) (end 154.453199 142.057999) (width 0.75) (layer B.Cu) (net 1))
 (segment (start 154.453199 142.057999) (end 155.028201 142.633001) (width 0.75) (layer B.Cu) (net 1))
 (segment (start 155.028201 142.633001) (end 155.7782 143.383) (width 0.75) (layer B.Cu) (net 1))
 (segment (start 155.7274 122.5042) (end 154.402399 123.829201) (width 0.75) (layer B.Cu) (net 1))
 (segment (start 154.402399 123.829201) (end 154.402399 131.432999) (width 0.75) (layer B.Cu) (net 1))
 (segment (start 154.402399 131.432999) (end 155.028201 132.058801) (width 0.75) (layer B.Cu) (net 1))
 (segment (start 155.028201 132.058801) (end 155.7782 132.8088) (width 0.75) (layer B.Cu) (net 1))
 (segment (start 153.924 118.89232) (end 153.924 120.7008) (width 0.75) (layer B.Cu) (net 1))
 (segment (start 153.924 120.7008) (end 155.7274 122.5042) (width 0.75) (layer B.Cu) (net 1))
 (segment (start 153.82748 118.7958) (end 153.924 118.89232) (width 0.4) (layer F.Cu) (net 1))
 (segment (start 133.3158 112.268) (end 134.03199 112.268) (width 0.4) (layer F.Cu) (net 16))
 (segment (start 134.03199 112.268) (end 139.8016 106.49839) (width 0.4) (layer F.Cu) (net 16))
 (segment (start 139.8016 106.49839) (end 139.8016 106.2482) (width 0.4) (layer F.Cu) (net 16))
 (segment (start 140.969574 108.09784) (end 141.569574 107.49784) (width 0.4) (layer F.Cu) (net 17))
 (segment (start 139.899233 108.097841) (end 140.969574 108.09784) (width 0.4) (layer F.Cu) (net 17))
 (segment (start 134.429074 113.568) (end 139.899233 108.097841) (width 0.4) (layer F.Cu) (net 17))
 (segment (start 133.3158 113.568) (end 134.429074 113.568) (width 0.4) (layer F.Cu) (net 17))
 (segment (start 141.569574 107.49784) (end 142.217105 107.49784) (width 0.4) (layer F.Cu) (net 17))
 (segment (start 142.217105 107.49784) (end 143.466745 106.2482) (width 0.4) (layer F.Cu) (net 17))
 (segment (start 143.466745 106.2482) (end 143.80464 106.2482) (width 0.4) (layer F.Cu) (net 17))
 (segment (start 134.230531 112.918) (end 139.6507 107.497831) (width 0.4) (layer F.Cu) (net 18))
 (segment (start 133.3158 112.918) (end 134.230531 112.918) (width 0.4) (layer F.Cu) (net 18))
 (segment (start 139.6507 107.497831) (end 140.721041 107.497831) (width 0.4) (layer F.Cu) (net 18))
 (segment (start 140.721041 107.497831) (end 141.80312 106.415752) (width 0.4) (layer F.Cu) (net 18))
 (segment (start 141.80312 106.415752) (end 141.80312 106.2482) (width 0.4) (layer F.Cu) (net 18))
 (segment (start 141.818105 108.097851) (end 142.465637 108.097851) (width 0.4) (layer F.Cu) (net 19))
 (segment (start 143.2306 107.6452) (end 144.65681 107.6452) (width 0.4) (layer F.Cu) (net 19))
 (segment (start 142.8242 108.0516) (end 143.2306 107.6452) (width 0.4) (layer F.Cu) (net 19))
 (segment (start 134.627616 114.218) (end 140.147766 108.69785) (width 0.4) (layer F.Cu) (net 19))
 (segment (start 133.3158 114.218) (end 134.627616 114.218) (width 0.4) (layer F.Cu) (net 19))
 (segment (start 141.218107 108.697849) (end 141.818105 108.097851) (width 0.4) (layer F.Cu) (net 19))
 (segment (start 140.147766 108.69785) (end 141.218107 108.697849) (width 0.4) (layer F.Cu) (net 19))
 (segment (start 142.465637 108.097851) (end 142.511888 108.0516) (width 0.4) (layer F.Cu) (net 19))
 (segment (start 142.511888 108.0516) (end 142.8242 108.0516) (width 0.4) (layer F.Cu) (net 19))
 (segment (start 144.65681 107.6452) (end 145.80362 106.49839) (width 0.4) (layer F.Cu) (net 19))
 (segment (start 145.80362 106.49839) (end 145.80362 106.2482) (width 0.4) (layer F.Cu) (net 19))
 (segment (start 145.502199 114.228401) (end 144.826199 113.552401) (width 0.4) (layer F.Cu) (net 20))
 (segment (start 155.7274 130.1242) (end 154.577399 128.974199) (width 0.4) (layer F.Cu) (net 20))
 (segment (start 144.826199 113.552401) (end 144.826199 112.417967) (width 0.4) (layer F.Cu) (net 20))
 (segment (start 144.826199 112.417967) (end 144.676232 112.268) (width 0.4) (layer F.Cu) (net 20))
 (segment (start 147.491832 114.228401) (end 145.502199 114.228401) (width 0.4) (layer F.Cu) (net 20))
 (segment (start 149.226234 116.784806) (end 149.226234 115.962803) (width 0.4) (layer F.Cu) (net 20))
 (segment (start 154.577399 122.135971) (end 149.226234 116.784806) (width 0.4) (layer F.Cu) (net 20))
 (segment (start 144.676232 112.268) (end 140.0158 112.268) (width 0.4) (layer F.Cu) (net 20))
 (segment (start 140.0158 112.268) (end 139.1158 112.268) (width 0.4) (layer F.Cu) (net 20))
 (segment (start 149.226234 115.962803) (end 147.491832 114.228401) (width 0.4) (layer F.Cu) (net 20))
 (segment (start 154.577399 128.974199) (end 154.577399 122.135971) (width 0.4) (layer F.Cu) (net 20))
 (segment (start 147.2433 114.828412) (end 148.626223 116.211335) (width 0.4) (layer F.Cu) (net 21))
 (segment (start 144.226188 113.017978) (end 144.226188 113.800933) (width 0.4) (layer F.Cu) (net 21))
 (segment (start 155.028201 139.678801) (end 155.7782 140.4288) (width 0.4) (layer F.Cu) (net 21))
 (segment (start 153.977388 138.627988) (end 155.028201 139.678801) (width 0.4) (layer F.Cu) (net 21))
 (segment (start 144.226188 113.800933) (end 145.253667 114.828412) (width 0.4) (layer F.Cu) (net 21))
 (segment (start 148.626223 116.211335) (end 148.626223 117.033338) (width 0.4) (layer F.Cu) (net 21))
 (segment (start 148.626223 117.033338) (end 153.977388 122.384503) (width 0.4) (layer F.Cu) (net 21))
 (segment (start 153.977388 122.384503) (end 153.977388 138.627988) (width 0.4) (layer F.Cu) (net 21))
 (segment (start 144.12621 112.918) (end 144.226188 113.017978) (width 0.4) (layer F.Cu) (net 21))
 (segment (start 139.1158 112.918) (end 144.12621 112.918) (width 0.4) (layer F.Cu) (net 21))
 (segment (start 145.253667 114.828412) (end 147.2433 114.828412) (width 0.4) (layer F.Cu) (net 21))
 (segment (start 155.028201 150.253001) (end 155.7782 151.003) (width 0.4) (layer F.Cu) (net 4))
 (segment (start 153.377377 148.602177) (end 155.028201 150.253001) (width 0.4) (layer F.Cu) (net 4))
 (segment (start 148.026212 117.28187) (end 153.377377 122.633035) (width 0.4) (layer F.Cu) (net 4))
 (segment (start 148.026212 116.459867) (end 148.026212 117.28187) (width 0.4) (layer F.Cu) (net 4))
 (segment (start 143.626177 114.049465) (end 145.005135 115.428423) (width 0.4) (layer F.Cu) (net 4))
 (segment (start 153.377377 122.633035) (end 153.377377 148.602177) (width 0.4) (layer F.Cu) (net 4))
 (segment (start 139.1158 113.568) (end 143.576188 113.568) (width 0.4) (layer F.Cu) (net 4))
 (segment (start 146.994768 115.428423) (end 148.026212 116.459867) (width 0.4) (layer F.Cu) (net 4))
 (segment (start 145.005135 115.428423) (end 146.994768 115.428423) (width 0.4) (layer F.Cu) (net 4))
 (segment (start 143.576188 113.568) (end 143.626177 113.617989) (width 0.4) (layer F.Cu) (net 4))
 (segment (start 143.626177 113.617989) (end 143.626177 114.049465) (width 0.4) (layer F.Cu) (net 4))
 (segment (start 155.829 161.4932) (end 152.777366 158.441566) (width 0.4) (layer F.Cu) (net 22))
 (segment (start 152.777366 122.881566) (end 147.426201 117.530401) (width 0.4) (layer F.Cu) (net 22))
 (segment (start 152.777366 158.441566) (end 152.777366 122.881566) (width 0.4) (layer F.Cu) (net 22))
 (segment (start 143.026166 114.218) (end 139.1158 114.218) (width 0.4) (layer F.Cu) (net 22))
 (segment (start 147.426201 117.530401) (end 147.426201 116.708399) (width 0.4) (layer F.Cu) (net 22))
 (segment (start 147.426201 116.708399) (end 146.746236 116.028434) (width 0.4) (layer F.Cu) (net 22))
 (segment (start 146.746236 116.028434) (end 144.756603 116.028434) (width 0.4) (layer F.Cu) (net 22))
 (segment (start 144.756603 116.028434) (end 143.026166 114.297997) (width 0.4) (layer F.Cu) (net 22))
 (segment (start 143.026166 114.297997) (end 143.026166 114.218) (width 0.4) (layer F.Cu) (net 22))
 (segment (start 145.4912 165.5826) (end 145.4912 167.18223) (width 0.75) (layer B.Cu) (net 9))
 (segment (start 132.103169 161.094681) (end 132.103169 158.975799) (width 0.75) (layer B.Cu) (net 9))
 (segment (start 145.4912 167.18223) (end 145.279752 167.393678) (width 0.75) (layer B.Cu) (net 9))
 (segment (start 145.279752 167.393678) (end 139.250478 167.393678) (width 0.75) (layer B.Cu) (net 9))
 (segment (start 138.3538 166.497) (end 138.3538 165.274998) (width 0.75) (layer B.Cu) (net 9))
 (segment (start 138.3538 165.274998) (end 134.419602 161.3408) (width 0.75) (layer B.Cu) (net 9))
 (segment (start 139.250478 167.393678) (end 138.3538 166.497) (width 0.75) (layer B.Cu) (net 9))
 (segment (start 134.419602 161.3408) (end 132.349288 161.3408) (width 0.75) (layer B.Cu) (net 9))
 (segment (start 132.349288 161.3408) (end 132.103169 161.094681) (width 0.75) (layer B.Cu) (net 9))
 (segment (start 132.103169 158.975799) (end 133.045248 158.03372) (width 0.75) (layer B.Cu) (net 9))
 (segment (start 133.045248 158.03372) (end 133.5278 158.03372) (width 0.75) (layer B.Cu) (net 9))
 (segment (start 133.6294 136.58088) (end 133.37921 136.58088) (width 0.75) (layer B.Cu) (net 9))
 (segment (start 133.37921 136.58088) (end 132.153969 135.355639) (width 0.75) (layer B.Cu) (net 9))
 (segment (start 132.153969 135.355639) (end 132.153969 127.235959) (width 0.75) (layer B.Cu) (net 9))
 (segment (start 132.153969 127.235959) (end 133.096048 126.29388) (width 0.75) (layer B.Cu) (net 9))
 (segment (start 133.096048 126.29388) (end 133.5786 126.29388) (width 0.75) (layer B.Cu) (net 9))
 (segment (start 133.6548 147.50288) (end 133.40461 147.50288) (width 0.75) (layer B.Cu) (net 9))
 (segment (start 133.40461 147.50288) (end 132.204769 146.303039) (width 0.75) (layer B.Cu) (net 9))
 (segment (start 132.204769 146.303039) (end 132.204769 137.522959) (width 0.75) (layer B.Cu) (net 9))
 (segment (start 132.204769 137.522959) (end 133.146848 136.58088) (width 0.75) (layer B.Cu) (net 9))
 (segment (start 133.146848 136.58088) (end 133.6294 136.58088) (width 0.75) (layer B.Cu) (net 9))
 (segment (start 133.5278 158.03372) (end 133.27761 158.03372) (width 0.75) (layer B.Cu) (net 9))
 (segment (start 132.10316 156.85927) (end 132.10316 148.571968) (width 0.75) (layer B.Cu) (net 9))
 (segment (start 133.27761 158.03372) (end 132.10316 156.85927) (width 0.75) (layer B.Cu) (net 9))
 (segment (start 132.10316 148.571968) (end 133.172248 147.50288) (width 0.75) (layer B.Cu) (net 9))
 (segment (start 133.172248 147.50288) (end 133.6548 147.50288) (width 0.75) (layer B.Cu) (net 9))
 (segment (start 150.095649 113.214849) (end 150.8674 113.214849) (width 0.4) (layer B.Cu) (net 2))
 (segment (start 150.8674 113.214849) (end 151.291664 113.214849) (width 0.4) (layer B.Cu) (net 2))
 (segment (start 150.0886 113.2078) (end 150.095649 113.214849) (width 0.4) (layer B.Cu) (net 2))
 (segment (start 151.298713 113.2078) (end 151.291664 113.214849) (width 0.4) (layer F.Cu) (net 2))
 (segment (start 152.48128 113.2078) (end 151.298713 113.2078) (width 0.4) (layer F.Cu) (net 2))
 (via (at 133.3754 117.5512) (size 0.6) (drill 0.4) (layers F.Cu B.Cu) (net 3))
 (via (at 139.1666 117.4496) (size 0.6) (drill 0.4) (layers F.Cu B.Cu) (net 1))
 (via (at 151.291664 113.214849) (size 0.6) (drill 0.4) (layers F.Cu B.Cu) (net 2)))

